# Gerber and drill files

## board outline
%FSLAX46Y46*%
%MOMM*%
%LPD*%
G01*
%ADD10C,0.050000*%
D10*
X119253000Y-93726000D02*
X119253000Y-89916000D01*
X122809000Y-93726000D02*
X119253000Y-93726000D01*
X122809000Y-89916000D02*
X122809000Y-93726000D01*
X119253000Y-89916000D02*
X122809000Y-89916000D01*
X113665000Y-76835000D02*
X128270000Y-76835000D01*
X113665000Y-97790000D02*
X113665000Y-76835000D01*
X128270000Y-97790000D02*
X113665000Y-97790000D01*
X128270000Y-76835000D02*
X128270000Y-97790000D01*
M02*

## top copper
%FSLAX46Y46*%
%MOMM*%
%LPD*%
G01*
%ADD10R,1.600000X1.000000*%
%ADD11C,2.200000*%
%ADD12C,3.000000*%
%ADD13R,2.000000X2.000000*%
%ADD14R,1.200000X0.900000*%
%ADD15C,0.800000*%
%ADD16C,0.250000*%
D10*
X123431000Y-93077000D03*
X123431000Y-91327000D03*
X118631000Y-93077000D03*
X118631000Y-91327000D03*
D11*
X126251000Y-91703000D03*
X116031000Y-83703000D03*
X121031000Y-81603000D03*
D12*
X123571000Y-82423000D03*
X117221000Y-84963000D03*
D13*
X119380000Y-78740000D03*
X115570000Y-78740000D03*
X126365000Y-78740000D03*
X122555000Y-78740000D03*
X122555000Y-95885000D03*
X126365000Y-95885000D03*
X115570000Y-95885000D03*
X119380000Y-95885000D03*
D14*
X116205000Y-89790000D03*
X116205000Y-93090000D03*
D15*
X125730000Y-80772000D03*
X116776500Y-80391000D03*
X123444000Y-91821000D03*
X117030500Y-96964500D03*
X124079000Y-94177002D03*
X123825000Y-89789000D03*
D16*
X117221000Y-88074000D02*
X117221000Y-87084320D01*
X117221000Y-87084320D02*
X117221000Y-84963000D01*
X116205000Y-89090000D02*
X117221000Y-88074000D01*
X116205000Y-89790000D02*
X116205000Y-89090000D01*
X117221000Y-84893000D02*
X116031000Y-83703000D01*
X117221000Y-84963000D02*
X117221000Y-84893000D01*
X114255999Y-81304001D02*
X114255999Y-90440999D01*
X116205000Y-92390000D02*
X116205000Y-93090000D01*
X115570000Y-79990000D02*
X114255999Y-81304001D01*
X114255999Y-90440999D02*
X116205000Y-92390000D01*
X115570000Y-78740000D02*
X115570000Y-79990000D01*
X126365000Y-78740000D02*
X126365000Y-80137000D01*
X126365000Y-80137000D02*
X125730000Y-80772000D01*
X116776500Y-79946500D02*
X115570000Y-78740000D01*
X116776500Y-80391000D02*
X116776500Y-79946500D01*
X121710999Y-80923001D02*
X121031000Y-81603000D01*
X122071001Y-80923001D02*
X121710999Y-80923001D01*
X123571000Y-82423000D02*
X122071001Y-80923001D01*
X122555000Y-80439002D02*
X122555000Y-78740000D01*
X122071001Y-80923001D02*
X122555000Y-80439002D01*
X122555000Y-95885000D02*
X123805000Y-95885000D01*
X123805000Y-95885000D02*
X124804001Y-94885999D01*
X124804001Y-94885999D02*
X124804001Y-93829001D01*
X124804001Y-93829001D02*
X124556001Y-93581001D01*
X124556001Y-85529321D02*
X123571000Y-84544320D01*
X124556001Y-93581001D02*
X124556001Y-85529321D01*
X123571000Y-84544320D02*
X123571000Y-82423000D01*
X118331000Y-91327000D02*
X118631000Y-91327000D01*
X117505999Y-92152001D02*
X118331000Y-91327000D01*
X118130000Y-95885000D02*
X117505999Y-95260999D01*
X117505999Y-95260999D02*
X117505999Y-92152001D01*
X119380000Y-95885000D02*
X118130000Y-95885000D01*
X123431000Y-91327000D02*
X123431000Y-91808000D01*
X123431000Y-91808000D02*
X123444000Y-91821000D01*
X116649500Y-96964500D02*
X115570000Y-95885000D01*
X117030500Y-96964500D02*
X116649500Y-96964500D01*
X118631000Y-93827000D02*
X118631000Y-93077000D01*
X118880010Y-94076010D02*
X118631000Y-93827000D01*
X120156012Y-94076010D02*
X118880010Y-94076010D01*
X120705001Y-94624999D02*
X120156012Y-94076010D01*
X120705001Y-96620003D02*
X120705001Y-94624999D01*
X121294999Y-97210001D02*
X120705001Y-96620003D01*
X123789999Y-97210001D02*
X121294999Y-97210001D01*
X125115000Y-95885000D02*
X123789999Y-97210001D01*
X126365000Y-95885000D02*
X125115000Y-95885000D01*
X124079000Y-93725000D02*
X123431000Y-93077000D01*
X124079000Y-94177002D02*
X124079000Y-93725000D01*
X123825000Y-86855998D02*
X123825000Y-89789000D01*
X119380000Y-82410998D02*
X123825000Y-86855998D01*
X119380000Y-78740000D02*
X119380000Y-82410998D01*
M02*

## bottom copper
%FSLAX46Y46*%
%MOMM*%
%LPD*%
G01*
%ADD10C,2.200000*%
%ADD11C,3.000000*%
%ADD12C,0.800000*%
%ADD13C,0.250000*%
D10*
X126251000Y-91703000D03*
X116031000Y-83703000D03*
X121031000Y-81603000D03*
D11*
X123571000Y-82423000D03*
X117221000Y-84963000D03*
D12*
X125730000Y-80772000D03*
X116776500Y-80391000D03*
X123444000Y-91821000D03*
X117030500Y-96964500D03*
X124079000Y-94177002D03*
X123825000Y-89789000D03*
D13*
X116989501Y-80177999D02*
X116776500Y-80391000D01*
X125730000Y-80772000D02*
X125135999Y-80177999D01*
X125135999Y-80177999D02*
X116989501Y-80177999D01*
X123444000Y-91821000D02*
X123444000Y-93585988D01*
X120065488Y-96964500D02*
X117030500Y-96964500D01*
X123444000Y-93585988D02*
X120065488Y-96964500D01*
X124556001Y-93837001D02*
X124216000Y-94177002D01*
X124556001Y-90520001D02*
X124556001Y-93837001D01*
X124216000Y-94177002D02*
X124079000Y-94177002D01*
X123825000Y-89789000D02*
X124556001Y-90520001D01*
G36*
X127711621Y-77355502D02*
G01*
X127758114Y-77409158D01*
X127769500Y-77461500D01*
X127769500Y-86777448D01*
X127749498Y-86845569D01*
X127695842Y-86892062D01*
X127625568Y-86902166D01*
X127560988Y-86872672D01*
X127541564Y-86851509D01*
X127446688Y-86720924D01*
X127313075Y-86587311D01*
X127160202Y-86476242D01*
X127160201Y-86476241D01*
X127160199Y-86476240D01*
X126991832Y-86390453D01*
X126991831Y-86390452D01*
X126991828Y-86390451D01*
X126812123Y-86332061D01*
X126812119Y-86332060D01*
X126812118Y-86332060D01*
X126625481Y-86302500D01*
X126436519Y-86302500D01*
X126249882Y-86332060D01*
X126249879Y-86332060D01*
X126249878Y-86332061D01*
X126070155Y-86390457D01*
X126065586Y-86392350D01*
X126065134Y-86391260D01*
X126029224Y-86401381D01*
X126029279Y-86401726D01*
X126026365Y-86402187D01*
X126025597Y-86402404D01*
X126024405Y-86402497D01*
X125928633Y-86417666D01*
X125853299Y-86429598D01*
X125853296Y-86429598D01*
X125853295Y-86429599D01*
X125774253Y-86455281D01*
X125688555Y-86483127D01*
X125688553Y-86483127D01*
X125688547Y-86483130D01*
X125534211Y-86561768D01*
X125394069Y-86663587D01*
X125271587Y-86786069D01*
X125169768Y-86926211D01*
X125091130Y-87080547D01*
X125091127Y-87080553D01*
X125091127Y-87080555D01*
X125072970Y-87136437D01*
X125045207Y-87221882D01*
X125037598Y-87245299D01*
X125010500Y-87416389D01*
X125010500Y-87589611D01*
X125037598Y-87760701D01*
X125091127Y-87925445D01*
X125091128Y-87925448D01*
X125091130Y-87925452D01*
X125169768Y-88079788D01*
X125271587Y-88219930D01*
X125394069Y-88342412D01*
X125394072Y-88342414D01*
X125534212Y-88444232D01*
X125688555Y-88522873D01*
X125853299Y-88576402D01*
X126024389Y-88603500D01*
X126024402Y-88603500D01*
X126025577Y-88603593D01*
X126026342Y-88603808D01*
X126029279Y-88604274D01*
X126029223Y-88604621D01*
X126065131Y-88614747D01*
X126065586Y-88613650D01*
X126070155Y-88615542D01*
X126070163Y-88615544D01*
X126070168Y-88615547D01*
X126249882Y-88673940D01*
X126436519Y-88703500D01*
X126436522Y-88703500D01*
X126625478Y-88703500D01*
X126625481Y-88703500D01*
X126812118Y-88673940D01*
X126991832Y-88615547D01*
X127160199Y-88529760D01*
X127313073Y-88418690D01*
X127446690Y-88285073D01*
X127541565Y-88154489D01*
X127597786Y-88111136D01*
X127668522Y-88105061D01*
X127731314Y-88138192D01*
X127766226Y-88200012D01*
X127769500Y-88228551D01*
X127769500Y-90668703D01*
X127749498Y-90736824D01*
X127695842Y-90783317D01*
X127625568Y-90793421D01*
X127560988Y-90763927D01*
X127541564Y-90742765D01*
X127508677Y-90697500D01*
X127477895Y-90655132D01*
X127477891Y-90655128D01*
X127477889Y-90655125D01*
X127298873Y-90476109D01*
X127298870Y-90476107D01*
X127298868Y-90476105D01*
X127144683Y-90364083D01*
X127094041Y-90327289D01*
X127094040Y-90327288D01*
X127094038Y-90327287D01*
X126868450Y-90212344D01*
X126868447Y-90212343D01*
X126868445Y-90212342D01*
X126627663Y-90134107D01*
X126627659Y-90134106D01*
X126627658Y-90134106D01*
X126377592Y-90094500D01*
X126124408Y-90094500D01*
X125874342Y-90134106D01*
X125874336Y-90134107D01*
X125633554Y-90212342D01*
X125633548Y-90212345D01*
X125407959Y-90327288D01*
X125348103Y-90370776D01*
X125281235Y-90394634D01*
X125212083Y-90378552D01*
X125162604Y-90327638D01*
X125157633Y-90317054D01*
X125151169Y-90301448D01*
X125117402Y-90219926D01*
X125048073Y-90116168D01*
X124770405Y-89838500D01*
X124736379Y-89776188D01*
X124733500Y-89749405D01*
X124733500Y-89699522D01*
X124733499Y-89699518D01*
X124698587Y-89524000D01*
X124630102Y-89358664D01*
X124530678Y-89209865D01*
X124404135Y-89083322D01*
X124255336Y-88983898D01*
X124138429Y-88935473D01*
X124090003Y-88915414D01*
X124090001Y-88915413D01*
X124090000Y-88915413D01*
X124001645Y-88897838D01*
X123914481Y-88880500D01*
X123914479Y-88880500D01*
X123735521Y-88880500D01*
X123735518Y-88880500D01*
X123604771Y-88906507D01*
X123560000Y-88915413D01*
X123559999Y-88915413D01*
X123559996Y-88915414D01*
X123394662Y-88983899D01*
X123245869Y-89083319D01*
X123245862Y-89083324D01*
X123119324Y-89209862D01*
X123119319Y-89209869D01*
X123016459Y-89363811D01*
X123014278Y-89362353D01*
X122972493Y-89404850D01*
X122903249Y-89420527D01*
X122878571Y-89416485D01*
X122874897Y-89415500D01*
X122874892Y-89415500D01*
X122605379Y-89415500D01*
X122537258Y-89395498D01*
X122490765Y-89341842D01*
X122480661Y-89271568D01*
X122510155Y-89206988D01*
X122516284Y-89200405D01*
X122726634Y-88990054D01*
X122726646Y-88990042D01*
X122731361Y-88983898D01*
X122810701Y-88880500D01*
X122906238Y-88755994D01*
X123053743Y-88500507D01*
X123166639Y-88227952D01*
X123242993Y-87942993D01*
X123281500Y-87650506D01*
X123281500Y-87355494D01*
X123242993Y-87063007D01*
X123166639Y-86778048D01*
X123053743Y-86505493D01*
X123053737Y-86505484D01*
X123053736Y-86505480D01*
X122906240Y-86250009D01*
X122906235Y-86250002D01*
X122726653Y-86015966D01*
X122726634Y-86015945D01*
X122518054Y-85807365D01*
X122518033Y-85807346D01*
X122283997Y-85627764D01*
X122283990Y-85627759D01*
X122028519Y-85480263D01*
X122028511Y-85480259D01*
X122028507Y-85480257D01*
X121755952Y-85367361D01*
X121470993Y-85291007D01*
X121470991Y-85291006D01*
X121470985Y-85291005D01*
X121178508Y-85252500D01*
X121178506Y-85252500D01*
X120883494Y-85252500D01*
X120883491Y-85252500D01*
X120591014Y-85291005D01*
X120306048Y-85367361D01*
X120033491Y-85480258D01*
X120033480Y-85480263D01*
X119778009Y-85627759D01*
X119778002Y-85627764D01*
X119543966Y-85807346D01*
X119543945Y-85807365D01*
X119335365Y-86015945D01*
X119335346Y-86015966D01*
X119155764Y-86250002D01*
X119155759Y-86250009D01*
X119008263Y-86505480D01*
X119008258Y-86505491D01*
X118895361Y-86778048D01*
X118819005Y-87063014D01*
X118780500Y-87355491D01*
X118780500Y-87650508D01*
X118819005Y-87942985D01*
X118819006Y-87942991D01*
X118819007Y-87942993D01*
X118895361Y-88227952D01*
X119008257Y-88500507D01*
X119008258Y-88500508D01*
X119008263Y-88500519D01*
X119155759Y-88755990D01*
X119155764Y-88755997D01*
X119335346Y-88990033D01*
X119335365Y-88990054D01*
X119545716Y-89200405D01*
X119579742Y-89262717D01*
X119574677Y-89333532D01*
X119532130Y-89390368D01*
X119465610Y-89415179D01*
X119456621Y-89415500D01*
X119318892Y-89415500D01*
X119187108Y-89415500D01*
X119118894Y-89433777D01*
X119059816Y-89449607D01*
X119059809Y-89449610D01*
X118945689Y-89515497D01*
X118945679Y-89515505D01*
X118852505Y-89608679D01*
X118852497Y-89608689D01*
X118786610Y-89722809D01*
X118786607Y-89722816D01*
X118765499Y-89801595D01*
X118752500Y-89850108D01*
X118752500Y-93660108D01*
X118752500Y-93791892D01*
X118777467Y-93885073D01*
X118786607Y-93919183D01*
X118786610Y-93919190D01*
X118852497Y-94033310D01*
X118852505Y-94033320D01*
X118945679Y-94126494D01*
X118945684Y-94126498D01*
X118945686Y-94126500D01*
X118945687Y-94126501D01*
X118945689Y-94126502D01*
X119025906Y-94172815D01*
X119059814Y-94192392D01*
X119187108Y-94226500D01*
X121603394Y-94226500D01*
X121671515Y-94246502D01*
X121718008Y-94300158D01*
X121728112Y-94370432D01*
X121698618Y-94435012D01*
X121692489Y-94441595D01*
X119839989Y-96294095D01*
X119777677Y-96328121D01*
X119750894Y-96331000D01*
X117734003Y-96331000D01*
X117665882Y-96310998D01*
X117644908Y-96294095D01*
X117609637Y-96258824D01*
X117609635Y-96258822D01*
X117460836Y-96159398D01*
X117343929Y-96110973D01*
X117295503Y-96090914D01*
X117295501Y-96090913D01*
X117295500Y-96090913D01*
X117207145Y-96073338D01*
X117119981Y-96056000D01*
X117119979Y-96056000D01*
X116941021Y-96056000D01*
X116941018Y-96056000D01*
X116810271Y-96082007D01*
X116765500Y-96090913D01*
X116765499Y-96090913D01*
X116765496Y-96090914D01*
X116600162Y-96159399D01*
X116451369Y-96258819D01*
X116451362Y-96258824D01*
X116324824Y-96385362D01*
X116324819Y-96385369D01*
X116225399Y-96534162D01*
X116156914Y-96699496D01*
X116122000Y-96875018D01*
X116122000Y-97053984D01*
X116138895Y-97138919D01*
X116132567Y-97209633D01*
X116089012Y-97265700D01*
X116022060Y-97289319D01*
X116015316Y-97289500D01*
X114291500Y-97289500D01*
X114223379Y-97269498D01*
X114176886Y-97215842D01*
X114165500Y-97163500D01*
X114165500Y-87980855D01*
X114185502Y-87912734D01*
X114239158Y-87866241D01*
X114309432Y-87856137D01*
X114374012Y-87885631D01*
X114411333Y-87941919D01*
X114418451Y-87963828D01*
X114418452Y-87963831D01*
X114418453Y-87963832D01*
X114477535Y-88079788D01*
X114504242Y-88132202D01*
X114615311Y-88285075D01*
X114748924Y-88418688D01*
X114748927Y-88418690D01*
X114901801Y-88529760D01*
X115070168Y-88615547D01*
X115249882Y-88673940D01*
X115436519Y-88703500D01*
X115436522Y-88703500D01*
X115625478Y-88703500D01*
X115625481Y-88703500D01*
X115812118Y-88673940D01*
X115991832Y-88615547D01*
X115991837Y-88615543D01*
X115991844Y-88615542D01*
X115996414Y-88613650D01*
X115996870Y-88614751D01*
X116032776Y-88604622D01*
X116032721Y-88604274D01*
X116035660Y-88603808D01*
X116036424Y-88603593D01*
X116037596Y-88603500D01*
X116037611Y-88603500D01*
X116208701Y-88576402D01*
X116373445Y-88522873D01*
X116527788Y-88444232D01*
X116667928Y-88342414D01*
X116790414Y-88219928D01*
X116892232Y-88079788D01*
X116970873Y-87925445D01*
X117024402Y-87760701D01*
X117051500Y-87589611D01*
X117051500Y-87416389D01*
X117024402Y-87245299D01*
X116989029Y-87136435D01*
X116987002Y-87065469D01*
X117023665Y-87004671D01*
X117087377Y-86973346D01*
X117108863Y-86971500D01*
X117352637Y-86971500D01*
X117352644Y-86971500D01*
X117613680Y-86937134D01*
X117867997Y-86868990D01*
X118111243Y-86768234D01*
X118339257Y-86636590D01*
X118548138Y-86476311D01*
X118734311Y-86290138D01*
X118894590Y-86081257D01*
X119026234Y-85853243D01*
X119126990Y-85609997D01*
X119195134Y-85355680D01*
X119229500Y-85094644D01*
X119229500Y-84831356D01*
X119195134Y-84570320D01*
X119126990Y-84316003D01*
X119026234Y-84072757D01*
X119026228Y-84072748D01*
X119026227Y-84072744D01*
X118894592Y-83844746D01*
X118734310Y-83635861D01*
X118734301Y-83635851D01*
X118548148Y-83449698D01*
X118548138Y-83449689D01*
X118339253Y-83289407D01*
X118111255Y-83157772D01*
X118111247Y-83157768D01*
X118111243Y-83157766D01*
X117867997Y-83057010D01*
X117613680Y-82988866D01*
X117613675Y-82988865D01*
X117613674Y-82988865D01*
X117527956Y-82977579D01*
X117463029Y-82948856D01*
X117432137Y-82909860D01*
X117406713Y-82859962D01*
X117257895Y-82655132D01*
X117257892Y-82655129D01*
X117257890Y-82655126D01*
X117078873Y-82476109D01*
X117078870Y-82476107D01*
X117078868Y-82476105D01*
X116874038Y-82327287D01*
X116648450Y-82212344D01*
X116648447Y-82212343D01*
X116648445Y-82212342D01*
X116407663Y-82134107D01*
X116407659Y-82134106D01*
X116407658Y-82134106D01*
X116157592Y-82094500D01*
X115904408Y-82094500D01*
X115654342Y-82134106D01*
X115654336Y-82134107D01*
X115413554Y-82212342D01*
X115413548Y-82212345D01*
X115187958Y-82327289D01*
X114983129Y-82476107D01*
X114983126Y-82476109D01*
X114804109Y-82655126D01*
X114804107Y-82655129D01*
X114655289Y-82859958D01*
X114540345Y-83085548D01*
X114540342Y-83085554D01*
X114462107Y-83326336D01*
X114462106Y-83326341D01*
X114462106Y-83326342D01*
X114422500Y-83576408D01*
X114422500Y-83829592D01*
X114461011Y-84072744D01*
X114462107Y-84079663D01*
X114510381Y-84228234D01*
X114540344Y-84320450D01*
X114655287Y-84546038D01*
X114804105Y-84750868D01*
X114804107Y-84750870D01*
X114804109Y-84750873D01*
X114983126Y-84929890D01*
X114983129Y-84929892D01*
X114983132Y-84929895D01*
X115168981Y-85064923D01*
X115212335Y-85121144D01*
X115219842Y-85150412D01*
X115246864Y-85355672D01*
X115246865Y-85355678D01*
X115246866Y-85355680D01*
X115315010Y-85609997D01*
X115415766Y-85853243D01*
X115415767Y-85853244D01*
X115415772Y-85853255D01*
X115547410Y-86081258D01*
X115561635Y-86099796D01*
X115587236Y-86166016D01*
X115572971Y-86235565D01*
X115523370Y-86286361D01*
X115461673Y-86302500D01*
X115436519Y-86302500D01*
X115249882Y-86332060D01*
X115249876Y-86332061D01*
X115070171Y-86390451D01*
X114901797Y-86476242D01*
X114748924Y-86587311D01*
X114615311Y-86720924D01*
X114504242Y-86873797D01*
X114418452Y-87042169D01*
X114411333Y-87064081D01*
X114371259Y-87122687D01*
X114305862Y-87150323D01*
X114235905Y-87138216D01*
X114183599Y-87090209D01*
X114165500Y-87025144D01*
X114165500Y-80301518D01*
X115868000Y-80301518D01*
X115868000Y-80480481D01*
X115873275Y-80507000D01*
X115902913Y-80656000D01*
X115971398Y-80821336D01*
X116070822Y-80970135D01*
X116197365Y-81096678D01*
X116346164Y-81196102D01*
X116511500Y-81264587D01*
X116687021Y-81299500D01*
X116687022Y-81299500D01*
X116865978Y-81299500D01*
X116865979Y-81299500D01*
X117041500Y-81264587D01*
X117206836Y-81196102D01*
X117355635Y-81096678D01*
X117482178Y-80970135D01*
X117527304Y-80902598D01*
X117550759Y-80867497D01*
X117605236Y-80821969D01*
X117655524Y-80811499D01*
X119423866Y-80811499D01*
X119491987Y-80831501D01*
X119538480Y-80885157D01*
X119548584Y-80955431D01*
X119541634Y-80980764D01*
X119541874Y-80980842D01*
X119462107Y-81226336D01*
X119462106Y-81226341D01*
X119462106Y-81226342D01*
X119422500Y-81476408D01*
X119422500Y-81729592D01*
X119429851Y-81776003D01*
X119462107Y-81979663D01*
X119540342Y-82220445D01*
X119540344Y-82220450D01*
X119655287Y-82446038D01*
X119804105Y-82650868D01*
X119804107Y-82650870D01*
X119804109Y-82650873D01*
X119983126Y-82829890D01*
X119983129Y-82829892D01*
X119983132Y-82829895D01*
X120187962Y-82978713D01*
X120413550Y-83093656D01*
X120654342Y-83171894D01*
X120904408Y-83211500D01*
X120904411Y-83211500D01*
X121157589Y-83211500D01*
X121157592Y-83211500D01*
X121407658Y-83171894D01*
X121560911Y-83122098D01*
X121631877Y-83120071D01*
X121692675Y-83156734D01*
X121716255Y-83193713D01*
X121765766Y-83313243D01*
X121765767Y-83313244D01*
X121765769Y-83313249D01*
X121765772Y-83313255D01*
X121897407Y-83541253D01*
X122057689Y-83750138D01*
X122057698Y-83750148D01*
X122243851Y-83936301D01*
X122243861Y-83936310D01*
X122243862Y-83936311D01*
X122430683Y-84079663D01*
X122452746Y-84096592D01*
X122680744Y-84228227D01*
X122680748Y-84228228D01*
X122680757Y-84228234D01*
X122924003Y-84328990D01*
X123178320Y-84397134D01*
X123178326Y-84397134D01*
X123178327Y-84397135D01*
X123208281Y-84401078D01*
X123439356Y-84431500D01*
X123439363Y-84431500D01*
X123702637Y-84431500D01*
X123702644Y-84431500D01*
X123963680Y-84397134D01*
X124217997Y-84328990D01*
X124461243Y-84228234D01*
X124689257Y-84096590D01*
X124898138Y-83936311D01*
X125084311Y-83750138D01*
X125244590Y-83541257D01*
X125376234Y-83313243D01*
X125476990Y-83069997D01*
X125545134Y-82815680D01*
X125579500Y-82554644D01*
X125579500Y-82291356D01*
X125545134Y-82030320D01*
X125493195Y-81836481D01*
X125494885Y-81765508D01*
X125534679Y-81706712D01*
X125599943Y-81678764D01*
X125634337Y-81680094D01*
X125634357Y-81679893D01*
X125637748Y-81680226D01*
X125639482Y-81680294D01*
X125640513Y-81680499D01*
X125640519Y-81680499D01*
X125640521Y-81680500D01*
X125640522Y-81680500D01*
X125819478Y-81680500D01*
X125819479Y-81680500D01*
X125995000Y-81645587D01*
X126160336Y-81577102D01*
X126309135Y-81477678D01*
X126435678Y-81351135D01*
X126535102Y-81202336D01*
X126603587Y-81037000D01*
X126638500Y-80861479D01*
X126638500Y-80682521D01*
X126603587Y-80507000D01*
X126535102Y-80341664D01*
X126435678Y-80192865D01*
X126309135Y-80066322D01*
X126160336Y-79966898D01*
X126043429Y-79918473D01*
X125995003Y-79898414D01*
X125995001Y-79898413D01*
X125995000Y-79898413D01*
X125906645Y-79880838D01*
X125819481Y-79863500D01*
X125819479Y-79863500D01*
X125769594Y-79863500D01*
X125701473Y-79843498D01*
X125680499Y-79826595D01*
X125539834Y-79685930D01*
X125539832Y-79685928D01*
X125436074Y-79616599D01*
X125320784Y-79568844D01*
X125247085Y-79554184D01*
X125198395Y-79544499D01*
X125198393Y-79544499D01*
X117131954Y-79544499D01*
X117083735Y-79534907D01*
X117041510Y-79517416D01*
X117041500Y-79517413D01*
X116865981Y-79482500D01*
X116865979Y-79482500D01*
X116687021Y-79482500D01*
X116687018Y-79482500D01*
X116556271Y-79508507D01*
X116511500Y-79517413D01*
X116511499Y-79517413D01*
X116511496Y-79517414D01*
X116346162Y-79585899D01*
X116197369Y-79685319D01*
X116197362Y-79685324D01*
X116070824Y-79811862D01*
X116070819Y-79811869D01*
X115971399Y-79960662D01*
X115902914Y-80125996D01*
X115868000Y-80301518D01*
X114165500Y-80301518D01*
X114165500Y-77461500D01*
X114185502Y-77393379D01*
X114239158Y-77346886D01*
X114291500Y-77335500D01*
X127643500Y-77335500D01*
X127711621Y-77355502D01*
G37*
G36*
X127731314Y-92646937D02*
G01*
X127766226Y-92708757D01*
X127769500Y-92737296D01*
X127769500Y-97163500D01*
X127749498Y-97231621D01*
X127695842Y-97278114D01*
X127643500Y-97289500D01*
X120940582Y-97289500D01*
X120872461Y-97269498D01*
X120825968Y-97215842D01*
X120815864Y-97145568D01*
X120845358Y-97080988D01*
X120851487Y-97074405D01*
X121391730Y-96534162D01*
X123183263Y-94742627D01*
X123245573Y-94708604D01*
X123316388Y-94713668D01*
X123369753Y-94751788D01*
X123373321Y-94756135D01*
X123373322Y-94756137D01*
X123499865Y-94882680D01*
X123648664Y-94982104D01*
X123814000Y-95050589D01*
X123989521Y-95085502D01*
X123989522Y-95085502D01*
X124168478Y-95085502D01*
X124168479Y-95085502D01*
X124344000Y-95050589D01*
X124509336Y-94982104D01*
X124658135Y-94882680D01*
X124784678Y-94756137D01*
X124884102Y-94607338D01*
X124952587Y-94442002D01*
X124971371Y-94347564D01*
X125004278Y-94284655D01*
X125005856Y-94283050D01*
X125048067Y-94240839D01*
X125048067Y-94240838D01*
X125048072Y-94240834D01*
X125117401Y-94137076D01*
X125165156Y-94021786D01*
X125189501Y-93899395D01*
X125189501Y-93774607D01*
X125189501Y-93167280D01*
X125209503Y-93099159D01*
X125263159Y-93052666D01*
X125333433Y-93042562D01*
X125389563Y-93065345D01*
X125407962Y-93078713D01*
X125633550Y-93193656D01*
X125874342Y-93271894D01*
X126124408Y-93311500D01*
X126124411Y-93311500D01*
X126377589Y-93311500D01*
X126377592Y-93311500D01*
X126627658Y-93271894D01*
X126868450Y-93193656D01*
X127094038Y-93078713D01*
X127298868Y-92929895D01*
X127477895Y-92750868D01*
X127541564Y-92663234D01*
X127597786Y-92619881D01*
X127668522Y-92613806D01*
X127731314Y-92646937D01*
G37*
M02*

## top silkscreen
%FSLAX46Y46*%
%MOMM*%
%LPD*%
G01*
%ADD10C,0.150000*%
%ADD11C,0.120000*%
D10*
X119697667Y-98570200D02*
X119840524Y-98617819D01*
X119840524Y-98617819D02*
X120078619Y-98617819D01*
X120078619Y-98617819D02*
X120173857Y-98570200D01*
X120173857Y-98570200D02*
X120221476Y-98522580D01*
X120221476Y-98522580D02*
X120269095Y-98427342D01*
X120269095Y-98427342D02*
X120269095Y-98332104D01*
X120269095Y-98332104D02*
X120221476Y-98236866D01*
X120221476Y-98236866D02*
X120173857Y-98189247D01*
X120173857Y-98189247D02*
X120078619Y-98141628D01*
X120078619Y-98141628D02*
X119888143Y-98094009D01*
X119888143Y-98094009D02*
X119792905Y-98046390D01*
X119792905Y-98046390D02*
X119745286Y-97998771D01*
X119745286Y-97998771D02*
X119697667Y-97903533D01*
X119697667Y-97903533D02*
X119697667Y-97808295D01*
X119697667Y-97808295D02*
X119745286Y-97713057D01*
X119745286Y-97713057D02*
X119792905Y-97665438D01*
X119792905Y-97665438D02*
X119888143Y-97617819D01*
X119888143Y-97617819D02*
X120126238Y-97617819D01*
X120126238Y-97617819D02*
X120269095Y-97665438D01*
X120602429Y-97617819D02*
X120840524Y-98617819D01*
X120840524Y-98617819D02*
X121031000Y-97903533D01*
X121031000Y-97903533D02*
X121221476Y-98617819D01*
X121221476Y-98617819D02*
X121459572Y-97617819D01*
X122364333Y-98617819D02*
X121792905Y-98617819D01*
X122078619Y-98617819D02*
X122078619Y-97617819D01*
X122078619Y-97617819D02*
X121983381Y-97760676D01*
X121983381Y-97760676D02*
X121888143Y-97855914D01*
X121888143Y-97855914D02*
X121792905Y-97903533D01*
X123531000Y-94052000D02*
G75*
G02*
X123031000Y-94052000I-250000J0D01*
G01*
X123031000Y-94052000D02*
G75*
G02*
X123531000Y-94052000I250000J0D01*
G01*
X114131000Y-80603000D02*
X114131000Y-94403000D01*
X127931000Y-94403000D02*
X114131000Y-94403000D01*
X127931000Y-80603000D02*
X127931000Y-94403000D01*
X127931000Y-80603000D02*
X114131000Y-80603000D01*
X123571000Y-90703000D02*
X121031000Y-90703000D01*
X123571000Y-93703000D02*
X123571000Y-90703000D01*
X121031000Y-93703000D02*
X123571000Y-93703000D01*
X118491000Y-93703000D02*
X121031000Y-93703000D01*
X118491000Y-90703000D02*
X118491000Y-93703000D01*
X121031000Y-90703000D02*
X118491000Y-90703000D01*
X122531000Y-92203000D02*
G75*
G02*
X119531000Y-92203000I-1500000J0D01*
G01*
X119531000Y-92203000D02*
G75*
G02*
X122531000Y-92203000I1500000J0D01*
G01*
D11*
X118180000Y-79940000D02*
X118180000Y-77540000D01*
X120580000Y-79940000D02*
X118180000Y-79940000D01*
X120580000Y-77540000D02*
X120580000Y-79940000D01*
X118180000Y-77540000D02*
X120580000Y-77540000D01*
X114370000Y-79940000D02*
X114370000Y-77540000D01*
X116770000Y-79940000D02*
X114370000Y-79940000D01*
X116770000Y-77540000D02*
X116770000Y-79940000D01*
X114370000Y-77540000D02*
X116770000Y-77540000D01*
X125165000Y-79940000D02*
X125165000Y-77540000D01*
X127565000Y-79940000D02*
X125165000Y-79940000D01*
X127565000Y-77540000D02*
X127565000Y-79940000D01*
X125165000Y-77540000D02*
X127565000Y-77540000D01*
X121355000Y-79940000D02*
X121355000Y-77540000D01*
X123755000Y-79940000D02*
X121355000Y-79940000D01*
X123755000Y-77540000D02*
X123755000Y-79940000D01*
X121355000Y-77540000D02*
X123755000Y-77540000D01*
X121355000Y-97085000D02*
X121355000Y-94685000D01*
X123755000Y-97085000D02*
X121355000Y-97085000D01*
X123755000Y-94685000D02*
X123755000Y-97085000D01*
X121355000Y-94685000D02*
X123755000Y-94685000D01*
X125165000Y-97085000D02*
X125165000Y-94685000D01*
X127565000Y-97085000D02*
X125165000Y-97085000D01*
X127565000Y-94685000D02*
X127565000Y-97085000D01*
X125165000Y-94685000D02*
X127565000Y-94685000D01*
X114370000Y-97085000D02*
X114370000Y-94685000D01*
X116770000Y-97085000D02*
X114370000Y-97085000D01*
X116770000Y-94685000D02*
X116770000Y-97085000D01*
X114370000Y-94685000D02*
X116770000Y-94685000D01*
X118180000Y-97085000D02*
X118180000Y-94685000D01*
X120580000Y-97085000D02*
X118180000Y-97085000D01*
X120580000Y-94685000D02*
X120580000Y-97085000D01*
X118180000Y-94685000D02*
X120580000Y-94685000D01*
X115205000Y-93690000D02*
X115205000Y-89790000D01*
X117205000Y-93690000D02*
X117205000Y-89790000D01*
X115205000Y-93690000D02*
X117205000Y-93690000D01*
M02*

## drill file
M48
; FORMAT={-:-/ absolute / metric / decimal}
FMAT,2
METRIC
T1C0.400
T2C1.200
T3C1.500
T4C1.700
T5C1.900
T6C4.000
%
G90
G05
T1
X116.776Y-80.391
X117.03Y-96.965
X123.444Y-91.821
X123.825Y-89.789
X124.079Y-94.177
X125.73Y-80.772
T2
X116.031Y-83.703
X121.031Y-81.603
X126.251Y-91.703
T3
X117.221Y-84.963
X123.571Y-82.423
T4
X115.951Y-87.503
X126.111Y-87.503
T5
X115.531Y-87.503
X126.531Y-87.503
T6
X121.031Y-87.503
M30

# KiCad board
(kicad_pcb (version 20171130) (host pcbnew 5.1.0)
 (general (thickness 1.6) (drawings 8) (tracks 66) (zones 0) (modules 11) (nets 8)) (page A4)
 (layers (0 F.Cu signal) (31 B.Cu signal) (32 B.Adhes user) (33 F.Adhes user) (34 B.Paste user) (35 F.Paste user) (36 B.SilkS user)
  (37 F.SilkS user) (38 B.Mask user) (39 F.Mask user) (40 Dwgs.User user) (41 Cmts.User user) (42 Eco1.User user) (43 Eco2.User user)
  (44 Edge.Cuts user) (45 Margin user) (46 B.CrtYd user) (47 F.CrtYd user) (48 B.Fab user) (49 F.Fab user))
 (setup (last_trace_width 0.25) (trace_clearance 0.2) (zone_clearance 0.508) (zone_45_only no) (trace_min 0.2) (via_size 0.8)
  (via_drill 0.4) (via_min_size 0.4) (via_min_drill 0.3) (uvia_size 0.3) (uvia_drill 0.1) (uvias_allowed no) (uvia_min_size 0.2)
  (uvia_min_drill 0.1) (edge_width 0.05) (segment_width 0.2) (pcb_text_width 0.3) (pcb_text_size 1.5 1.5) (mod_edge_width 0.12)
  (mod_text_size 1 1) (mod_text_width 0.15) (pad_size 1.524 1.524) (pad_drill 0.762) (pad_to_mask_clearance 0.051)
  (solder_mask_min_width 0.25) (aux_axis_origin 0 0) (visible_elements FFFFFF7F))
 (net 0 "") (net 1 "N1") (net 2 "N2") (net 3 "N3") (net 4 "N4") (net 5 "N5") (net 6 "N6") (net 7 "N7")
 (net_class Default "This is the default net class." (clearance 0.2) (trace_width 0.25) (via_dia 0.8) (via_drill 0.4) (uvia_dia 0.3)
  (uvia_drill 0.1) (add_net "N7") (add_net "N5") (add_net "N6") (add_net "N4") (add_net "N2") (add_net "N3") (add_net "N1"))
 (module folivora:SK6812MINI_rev (layer F.Cu) (at 121.031 92.202)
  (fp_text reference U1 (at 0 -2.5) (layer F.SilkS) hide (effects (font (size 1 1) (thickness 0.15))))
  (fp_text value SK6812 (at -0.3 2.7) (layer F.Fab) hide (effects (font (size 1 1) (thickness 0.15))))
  (fp_circle (center 2.25 1.85) (end 2.25 1.6) (layer F.SilkS) (width 0.15))
  (pad 4 smd rect (at 2.4 0.875) (size 1.6 1) (layers F.Cu F.Paste F.Mask) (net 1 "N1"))
  (pad 3 smd rect (at 2.4 -0.875) (size 1.6 1) (layers F.Cu F.Paste F.Mask) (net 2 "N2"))
  (pad 1 smd rect (at -2.4 0.875) (size 1.6 1) (layers F.Cu F.Paste F.Mask) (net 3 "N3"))
  (pad 2 smd rect (at -2.4 -0.875) (size 1.6 1) (layers F.Cu F.Paste F.Mask) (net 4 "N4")))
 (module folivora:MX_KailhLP (layer F.Cu) (at 121.031 87.503)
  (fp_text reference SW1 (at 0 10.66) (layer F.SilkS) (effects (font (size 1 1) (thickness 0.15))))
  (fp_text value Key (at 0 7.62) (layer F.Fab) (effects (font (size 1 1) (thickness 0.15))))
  (fp_line (start -6.9 -6.9) (end -6.9 6.9) (layer F.SilkS) (width 0.15))
  (fp_line (start 6.9 6.9) (end -6.9 6.9) (layer F.SilkS) (width 0.15))
  (fp_line (start 6.9 -6.9) (end 6.9 6.9) (layer F.SilkS) (width 0.15))
  (fp_line (start 6.9 -6.9) (end -6.9 -6.9) (layer F.SilkS) (width 0.15))
  (fp_line (start 2.54 3.2) (end 0 3.2) (layer F.SilkS) (width 0.15))
  (fp_line (start 2.54 6.2) (end 2.54 3.2) (layer F.SilkS) (width 0.15))
  (fp_line (start 0 6.2) (end 2.54 6.2) (layer F.SilkS) (width 0.15))
  (fp_line (start -2.54 6.2) (end 0 6.2) (layer F.SilkS) (width 0.15))
  (fp_line (start -2.54 3.2) (end -2.54 6.2) (layer F.SilkS) (width 0.15))
  (fp_line (start 0 3.2) (end -2.54 3.2) (layer F.SilkS) (width 0.15))
  (fp_circle (center 0 4.7) (end 1.5 4.7) (layer F.SilkS) (width 0.15))
  (pad "" thru_hole circle (at 5.22 4.2) (size 2.2 2.2) (drill 1.2) (layers *.Cu *.Mask))
  (pad 1 thru_hole circle (at -5 -3.8) (size 2.2 2.2) (drill 1.2) (layers *.Cu *.Mask) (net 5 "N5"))
  (pad 2 thru_hole circle (at 0 -5.9) (size 2.2 2.2) (drill 1.2) (layers *.Cu *.Mask) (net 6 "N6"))
  (pad "" np_thru_hole circle (at -5.5 0) (size 1.9 1.9) (drill 1.9) (layers *.Cu *.Mask))
  (pad "" np_thru_hole circle (at 5.5 0) (size 1.9 1.9) (drill 1.9) (layers *.Cu *.Mask))
  (pad 2 thru_hole circle (at 2.54 -5.08) (size 3 3) (drill 1.5) (layers *.Cu *.Mask) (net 6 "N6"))
  (pad 1 thru_hole circle (at -3.81 -2.54) (size 3 3) (drill 1.5) (layers *.Cu *.Mask) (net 5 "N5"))
  (pad "" np_thru_hole circle (at 5.08 0) (size 1.7 1.7) (drill 1.7) (layers *.Cu *.Mask))
  (pad "" np_thru_hole circle (at -5.08 0) (size 1.7 1.7) (drill 1.7) (layers *.Cu *.Mask))
  (pad "" np_thru_hole circle (at 0 0) (size 4 4) (drill 4) (layers *.Cu *.Mask)))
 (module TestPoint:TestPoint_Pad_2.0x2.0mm (layer F.Cu) (at 119.38 78.74)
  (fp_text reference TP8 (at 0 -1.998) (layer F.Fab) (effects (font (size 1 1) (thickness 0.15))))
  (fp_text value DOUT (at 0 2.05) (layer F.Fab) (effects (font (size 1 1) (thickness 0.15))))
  (fp_line (start -1.2 1.2) (end -1.2 -1.2) (layer F.SilkS) (width 0.12))
  (fp_line (start 1.2 1.2) (end -1.2 1.2) (layer F.SilkS) (width 0.12))
  (fp_line (start 1.2 -1.2) (end 1.2 1.2) (layer F.SilkS) (width 0.12))
  (fp_line (start -1.2 -1.2) (end 1.2 -1.2) (layer F.SilkS) (width 0.12))
  (pad 1 smd rect (at 0 0) (size 2 2) (layers F.Cu F.Mask) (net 1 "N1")))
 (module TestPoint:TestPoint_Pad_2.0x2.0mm (layer F.Cu) (at 115.57 78.74)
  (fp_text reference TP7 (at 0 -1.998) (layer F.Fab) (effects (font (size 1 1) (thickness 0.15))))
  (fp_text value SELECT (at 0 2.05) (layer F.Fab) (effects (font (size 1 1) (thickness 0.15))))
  (fp_line (start -1.2 1.2) (end -1.2 -1.2) (layer F.SilkS) (width 0.12))
  (fp_line (start 1.2 1.2) (end -1.2 1.2) (layer F.SilkS) (width 0.12))
  (fp_line (start 1.2 -1.2) (end 1.2 1.2) (layer F.SilkS) (width 0.12))
  (fp_line (start -1.2 -1.2) (end 1.2 -1.2) (layer F.SilkS) (width 0.12))
  (pad 1 smd rect (at 0 0) (size 2 2) (layers F.Cu F.Mask) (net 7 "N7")))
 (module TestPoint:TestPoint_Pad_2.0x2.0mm (layer F.Cu) (at 126.365 78.74)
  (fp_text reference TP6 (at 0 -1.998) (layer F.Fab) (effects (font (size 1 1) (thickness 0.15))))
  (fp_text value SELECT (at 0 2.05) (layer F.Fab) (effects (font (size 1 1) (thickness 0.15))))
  (fp_line (start -1.2 1.2) (end -1.2 -1.2) (layer F.SilkS) (width 0.12))
  (fp_line (start 1.2 1.2) (end -1.2 1.2) (layer F.SilkS) (width 0.12))
  (fp_line (start 1.2 -1.2) (end 1.2 1.2) (layer F.SilkS) (width 0.12))
  (fp_line (start -1.2 -1.2) (end 1.2 -1.2) (layer F.SilkS) (width 0.12))
  (pad 1 smd rect (at 0 0) (size 2 2) (layers F.Cu F.Mask) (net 7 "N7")))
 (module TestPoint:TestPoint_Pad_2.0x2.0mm (layer F.Cu) (at 122.555 78.74)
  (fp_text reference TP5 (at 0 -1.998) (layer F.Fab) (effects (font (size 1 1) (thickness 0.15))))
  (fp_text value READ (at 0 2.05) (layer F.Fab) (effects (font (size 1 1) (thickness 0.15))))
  (fp_line (start -1.2 1.2) (end -1.2 -1.2) (layer F.SilkS) (width 0.12))
  (fp_line (start 1.2 1.2) (end -1.2 1.2) (layer F.SilkS) (width 0.12))
  (fp_line (start 1.2 -1.2) (end 1.2 1.2) (layer F.SilkS) (width 0.12))
  (fp_line (start -1.2 -1.2) (end 1.2 -1.2) (layer F.SilkS) (width 0.12))
  (pad 1 smd rect (at 0 0) (size 2 2) (layers F.Cu F.Mask) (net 6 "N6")))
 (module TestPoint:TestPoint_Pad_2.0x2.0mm (layer F.Cu) (at 122.555 95.885)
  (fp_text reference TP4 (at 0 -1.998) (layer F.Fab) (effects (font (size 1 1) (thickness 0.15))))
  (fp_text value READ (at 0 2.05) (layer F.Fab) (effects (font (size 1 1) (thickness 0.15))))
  (fp_line (start -1.2 1.2) (end -1.2 -1.2) (layer F.SilkS) (width 0.12))
  (fp_line (start 1.2 1.2) (end -1.2 1.2) (layer F.SilkS) (width 0.12))
  (fp_line (start 1.2 -1.2) (end 1.2 1.2) (layer F.SilkS) (width 0.12))
  (fp_line (start -1.2 -1.2) (end 1.2 -1.2) (layer F.SilkS) (width 0.12))
  (pad 1 smd rect (at 0 0) (size 2 2) (layers F.Cu F.Mask) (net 6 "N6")))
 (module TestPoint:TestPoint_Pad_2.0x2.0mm (layer F.Cu) (at 126.365 95.885)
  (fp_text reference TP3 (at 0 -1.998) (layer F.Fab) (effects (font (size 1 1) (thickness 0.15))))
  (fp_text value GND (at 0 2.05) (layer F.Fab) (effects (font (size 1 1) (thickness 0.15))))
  (fp_line (start -1.2 1.2) (end -1.2 -1.2) (layer F.SilkS) (width 0.12))
  (fp_line (start 1.2 1.2) (end -1.2 1.2) (layer F.SilkS) (width 0.12))
  (fp_line (start 1.2 -1.2) (end 1.2 1.2) (layer F.SilkS) (width 0.12))
  (fp_line (start -1.2 -1.2) (end 1.2 -1.2) (layer F.SilkS) (width 0.12))
  (pad 1 smd rect (at 0 0) (size 2 2) (layers F.Cu F.Mask) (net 3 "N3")))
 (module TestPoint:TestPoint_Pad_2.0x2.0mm (layer F.Cu) (at 115.57 95.885)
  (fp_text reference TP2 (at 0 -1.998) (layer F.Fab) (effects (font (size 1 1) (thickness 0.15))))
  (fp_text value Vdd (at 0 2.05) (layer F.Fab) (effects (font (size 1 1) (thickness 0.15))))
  (fp_line (start -1.2 1.2) (end -1.2 -1.2) (layer F.SilkS) (width 0.12))
  (fp_line (start 1.2 1.2) (end -1.2 1.2) (layer F.SilkS) (width 0.12))
  (fp_line (start 1.2 -1.2) (end 1.2 1.2) (layer F.SilkS) (width 0.12))
  (fp_line (start -1.2 -1.2) (end 1.2 -1.2) (layer F.SilkS) (width 0.12))
  (pad 1 smd rect (at 0 0) (size 2 2) (layers F.Cu F.Mask) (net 2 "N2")))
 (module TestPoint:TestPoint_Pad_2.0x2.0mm (layer F.Cu) (at 119.38 95.885)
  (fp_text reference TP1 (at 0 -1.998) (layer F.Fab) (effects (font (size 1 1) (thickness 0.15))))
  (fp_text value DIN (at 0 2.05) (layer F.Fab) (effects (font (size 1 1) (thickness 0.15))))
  (fp_line (start -1.2 1.2) (end -1.2 -1.2) (layer F.SilkS) (width 0.12))
  (fp_line (start 1.2 1.2) (end -1.2 1.2) (layer F.SilkS) (width 0.12))
  (fp_line (start 1.2 -1.2) (end 1.2 1.2) (layer F.SilkS) (width 0.12))
  (fp_line (start -1.2 -1.2) (end 1.2 -1.2) (layer F.SilkS) (width 0.12))
  (pad 1 smd rect (at 0 0) (size 2 2) (layers F.Cu F.Mask) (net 4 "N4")))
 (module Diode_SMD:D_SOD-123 (layer F.Cu) (at 116.205 91.44 90)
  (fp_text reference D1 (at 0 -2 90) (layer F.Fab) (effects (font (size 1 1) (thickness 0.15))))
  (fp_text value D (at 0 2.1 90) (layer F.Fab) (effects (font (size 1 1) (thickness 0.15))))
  (fp_line (start -2.25 -1) (end 1.65 -1) (layer F.SilkS) (width 0.12))
  (fp_line (start -2.25 1) (end 1.65 1) (layer F.SilkS) (width 0.12))
  (fp_line (start -2.25 -1) (end -2.25 1) (layer F.SilkS) (width 0.12))
  (pad 2 smd rect (at 1.65 0 90) (size 0.9 1.2) (layers F.Cu F.Paste F.Mask) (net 5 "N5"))
  (pad 1 smd rect (at -1.65 0 90) (size 0.9 1.2) (layers F.Cu F.Paste F.Mask) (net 7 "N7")))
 (gr_line (start 119.253 93.726) (end 119.253 89.916) (layer Edge.Cuts) (width 0.05))
 (gr_line (start 122.809 93.726) (end 119.253 93.726) (layer Edge.Cuts) (width 0.05))
 (gr_line (start 122.809 89.916) (end 122.809 93.726) (layer Edge.Cuts) (width 0.05))
 (gr_line (start 119.253 89.916) (end 122.809 89.916) (layer Edge.Cuts) (width 0.05))
 (gr_line (start 113.665 76.835) (end 128.27 76.835) (layer Edge.Cuts) (width 0.05))
 (gr_line (start 113.665 97.79) (end 113.665 76.835) (layer Edge.Cuts) (width 0.05))
 (gr_line (start 128.27 97.79) (end 113.665 97.79) (layer Edge.Cuts) (width 0.05))
 (gr_line (start 128.27 76.835) (end 128.27 97.79) (layer Edge.Cuts) (width 0.05))
 (segment (start 117.221 88.074) (end 117.221 87.08432) (width 0.25) (layer F.Cu) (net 5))
 (segment (start 117.221 87.08432) (end 117.221 84.963) (width 0.25) (layer F.Cu) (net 5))
 (segment (start 116.205 89.09) (end 117.221 88.074) (width 0.25) (layer F.Cu) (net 5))
 (segment (start 116.205 89.79) (end 116.205 89.09) (width 0.25) (layer F.Cu) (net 5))
 (segment (start 117.221 84.893) (end 116.031 83.703) (width 0.25) (layer F.Cu) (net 5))
 (segment (start 117.221 84.963) (end 117.221 84.893) (width 0.25) (layer F.Cu) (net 5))
 (segment (start 114.255999 81.304001) (end 114.255999 90.440999) (width 0.25) (layer F.Cu) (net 7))
 (segment (start 116.205 92.39) (end 116.205 93.09) (width 0.25) (layer F.Cu) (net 7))
 (segment (start 115.57 79.99) (end 114.255999 81.304001) (width 0.25) (layer F.Cu) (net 7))
 (segment (start 114.255999 90.440999) (end 116.205 92.39) (width 0.25) (layer F.Cu) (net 7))
 (segment (start 115.57 78.74) (end 115.57 79.99) (width 0.25) (layer F.Cu) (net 7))
 (via (at 125.73 80.772) (size 0.8) (drill 0.4) (layers F.Cu B.Cu) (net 7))
 (segment (start 126.365 78.74) (end 126.365 80.137) (width 0.25) (layer F.Cu) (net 7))
 (segment (start 126.365 80.137) (end 125.73 80.772) (width 0.25) (layer F.Cu) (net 7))
 (via (at 116.7765 80.391) (size 0.8) (drill 0.4) (layers F.Cu B.Cu) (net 7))
 (segment (start 116.989501 80.177999) (end 116.7765 80.391) (width 0.25) (layer B.Cu) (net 7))
 (segment (start 125.73 80.772) (end 125.135999 80.177999) (width 0.25) (layer B.Cu) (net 7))
 (segment (start 125.135999 80.177999) (end 116.989501 80.177999) (width 0.25) (layer B.Cu) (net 7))
 (segment (start 116.7765 79.9465) (end 115.57 78.74) (width 0.25) (layer F.Cu) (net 7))
 (segment (start 116.7765 80.391) (end 116.7765 79.9465) (width 0.25) (layer F.Cu) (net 7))
 (segment (start 121.710999 80.923001) (end 121.031 81.603) (width 0.25) (layer F.Cu) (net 6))
 (segment (start 122.071001 80.923001) (end 121.710999 80.923001) (width 0.25) (layer F.Cu) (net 6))
 (segment (start 123.571 82.423) (end 122.071001 80.923001) (width 0.25) (layer F.Cu) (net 6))
 (segment (start 122.555 80.439002) (end 122.555 78.74) (width 0.25) (layer F.Cu) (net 6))
 (segment (start 122.071001 80.923001) (end 122.555 80.439002) (width 0.25) (layer F.Cu) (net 6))
 (segment (start 122.555 95.885) (end 123.805 95.885) (width 0.25) (layer F.Cu) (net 6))
 (segment (start 123.805 95.885) (end 124.804001 94.885999) (width 0.25) (layer F.Cu) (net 6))
 (segment (start 124.804001 94.885999) (end 124.804001 93.829001) (width 0.25) (layer F.Cu) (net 6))
 (segment (start 124.804001 93.829001) (end 124.556001 93.581001) (width 0.25) (layer F.Cu) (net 6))
 (segment (start 124.556001 85.529321) (end 123.571 84.54432) (width 0.25) (layer F.Cu) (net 6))
 (segment (start 124.556001 93.581001) (end 124.556001 85.529321) (width 0.25) (layer F.Cu) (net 6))
 (segment (start 123.571 84.54432) (end 123.571 82.423) (width 0.25) (layer F.Cu) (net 6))
 (segment (start 118.331 91.327) (end 118.631 91.327) (width 0.25) (layer F.Cu) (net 4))
 (segment (start 117.505999 92.152001) (end 118.331 91.327) (width 0.25) (layer F.Cu) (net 4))
 (segment (start 118.13 95.885) (end 117.505999 95.260999) (width 0.25) (layer F.Cu) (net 4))
 (segment (start 117.505999 95.260999) (end 117.505999 92.152001) (width 0.25) (layer F.Cu) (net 4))
 (segment (start 119.38 95.885) (end 118.13 95.885) (width 0.25) (layer F.Cu) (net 4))
 (via (at 123.444 91.821) (size 0.8) (drill 0.4) (layers F.Cu B.Cu) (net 2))
 (segment (start 123.431 91.327) (end 123.431 91.808) (width 0.25) (layer F.Cu) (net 2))
 (segment (start 123.431 91.808) (end 123.444 91.821) (width 0.25) (layer F.Cu) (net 2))
 (via (at 117.0305 96.9645) (size 0.8) (drill 0.4) (layers F.Cu B.Cu) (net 2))
 (segment (start 123.444 91.821) (end 123.444 93.585988) (width 0.25) (layer B.Cu) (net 2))
 (segment (start 120.065488 96.9645) (end 117.0305 96.9645) (width 0.25) (layer B.Cu) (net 2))
 (segment (start 123.444 93.585988) (end 120.065488 96.9645) (width 0.25) (layer B.Cu) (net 2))
 (segment (start 116.6495 96.9645) (end 115.57 95.885) (width 0.25) (layer F.Cu) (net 2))
 (segment (start 117.0305 96.9645) (end 116.6495 96.9645) (width 0.25) (layer F.Cu) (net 2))
 (segment (start 118.631 93.827) (end 118.631 93.077) (width 0.25) (layer F.Cu) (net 3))
 (segment (start 118.88001 94.07601) (end 118.631 93.827) (width 0.25) (layer F.Cu) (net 3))
 (segment (start 120.156012 94.07601) (end 118.88001 94.07601) (width 0.25) (layer F.Cu) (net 3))
 (segment (start 120.705001 94.624999) (end 120.156012 94.07601) (width 0.25) (layer F.Cu) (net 3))
 (segment (start 120.705001 96.620003) (end 120.705001 94.624999) (width 0.25) (layer F.Cu) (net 3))
 (segment (start 121.294999 97.210001) (end 120.705001 96.620003) (width 0.25) (layer F.Cu) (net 3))
 (segment (start 123.789999 97.210001) (end 121.294999 97.210001) (width 0.25) (layer F.Cu) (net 3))
 (segment (start 125.115 95.885) (end 123.789999 97.210001) (width 0.25) (layer F.Cu) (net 3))
 (segment (start 126.365 95.885) (end 125.115 95.885) (width 0.25) (layer F.Cu) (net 3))
 (via (at 124.079 94.177002) (size 0.8) (drill 0.4) (layers F.Cu B.Cu) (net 1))
 (segment (start 124.079 93.725) (end 123.431 93.077) (width 0.25) (layer F.Cu) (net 1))
 (segment (start 124.079 94.177002) (end 124.079 93.725) (width 0.25) (layer F.Cu) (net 1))
 (segment (start 124.556001 93.837001) (end 124.216 94.177002) (width 0.25) (layer B.Cu) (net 1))
 (segment (start 123.825 86.855998) (end 123.825 89.789) (width 0.25) (layer F.Cu) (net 1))
 (segment (start 119.38 82.410998) (end 123.825 86.855998) (width 0.25) (layer F.Cu) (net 1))
 (segment (start 124.556001 90.520001) (end 124.556001 93.837001) (width 0.25) (layer B.Cu) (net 1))
 (via (at 123.825 89.789) (size 0.8) (drill 0.4) (layers F.Cu B.Cu) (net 1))
 (segment (start 124.216 94.177002) (end 124.079 94.177002) (width 0.25) (layer B.Cu) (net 1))
 (segment (start 119.38 78.74) (end 119.38 82.410998) (width 0.25) (layer F.Cu) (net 1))
 (segment (start 123.825 89.789) (end 124.556001 90.520001) (width 0.25) (layer B.Cu) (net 1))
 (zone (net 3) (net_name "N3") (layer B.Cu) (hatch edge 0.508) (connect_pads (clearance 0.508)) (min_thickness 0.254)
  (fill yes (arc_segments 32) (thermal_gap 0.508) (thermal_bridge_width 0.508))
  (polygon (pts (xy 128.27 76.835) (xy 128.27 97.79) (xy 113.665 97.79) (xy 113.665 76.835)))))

